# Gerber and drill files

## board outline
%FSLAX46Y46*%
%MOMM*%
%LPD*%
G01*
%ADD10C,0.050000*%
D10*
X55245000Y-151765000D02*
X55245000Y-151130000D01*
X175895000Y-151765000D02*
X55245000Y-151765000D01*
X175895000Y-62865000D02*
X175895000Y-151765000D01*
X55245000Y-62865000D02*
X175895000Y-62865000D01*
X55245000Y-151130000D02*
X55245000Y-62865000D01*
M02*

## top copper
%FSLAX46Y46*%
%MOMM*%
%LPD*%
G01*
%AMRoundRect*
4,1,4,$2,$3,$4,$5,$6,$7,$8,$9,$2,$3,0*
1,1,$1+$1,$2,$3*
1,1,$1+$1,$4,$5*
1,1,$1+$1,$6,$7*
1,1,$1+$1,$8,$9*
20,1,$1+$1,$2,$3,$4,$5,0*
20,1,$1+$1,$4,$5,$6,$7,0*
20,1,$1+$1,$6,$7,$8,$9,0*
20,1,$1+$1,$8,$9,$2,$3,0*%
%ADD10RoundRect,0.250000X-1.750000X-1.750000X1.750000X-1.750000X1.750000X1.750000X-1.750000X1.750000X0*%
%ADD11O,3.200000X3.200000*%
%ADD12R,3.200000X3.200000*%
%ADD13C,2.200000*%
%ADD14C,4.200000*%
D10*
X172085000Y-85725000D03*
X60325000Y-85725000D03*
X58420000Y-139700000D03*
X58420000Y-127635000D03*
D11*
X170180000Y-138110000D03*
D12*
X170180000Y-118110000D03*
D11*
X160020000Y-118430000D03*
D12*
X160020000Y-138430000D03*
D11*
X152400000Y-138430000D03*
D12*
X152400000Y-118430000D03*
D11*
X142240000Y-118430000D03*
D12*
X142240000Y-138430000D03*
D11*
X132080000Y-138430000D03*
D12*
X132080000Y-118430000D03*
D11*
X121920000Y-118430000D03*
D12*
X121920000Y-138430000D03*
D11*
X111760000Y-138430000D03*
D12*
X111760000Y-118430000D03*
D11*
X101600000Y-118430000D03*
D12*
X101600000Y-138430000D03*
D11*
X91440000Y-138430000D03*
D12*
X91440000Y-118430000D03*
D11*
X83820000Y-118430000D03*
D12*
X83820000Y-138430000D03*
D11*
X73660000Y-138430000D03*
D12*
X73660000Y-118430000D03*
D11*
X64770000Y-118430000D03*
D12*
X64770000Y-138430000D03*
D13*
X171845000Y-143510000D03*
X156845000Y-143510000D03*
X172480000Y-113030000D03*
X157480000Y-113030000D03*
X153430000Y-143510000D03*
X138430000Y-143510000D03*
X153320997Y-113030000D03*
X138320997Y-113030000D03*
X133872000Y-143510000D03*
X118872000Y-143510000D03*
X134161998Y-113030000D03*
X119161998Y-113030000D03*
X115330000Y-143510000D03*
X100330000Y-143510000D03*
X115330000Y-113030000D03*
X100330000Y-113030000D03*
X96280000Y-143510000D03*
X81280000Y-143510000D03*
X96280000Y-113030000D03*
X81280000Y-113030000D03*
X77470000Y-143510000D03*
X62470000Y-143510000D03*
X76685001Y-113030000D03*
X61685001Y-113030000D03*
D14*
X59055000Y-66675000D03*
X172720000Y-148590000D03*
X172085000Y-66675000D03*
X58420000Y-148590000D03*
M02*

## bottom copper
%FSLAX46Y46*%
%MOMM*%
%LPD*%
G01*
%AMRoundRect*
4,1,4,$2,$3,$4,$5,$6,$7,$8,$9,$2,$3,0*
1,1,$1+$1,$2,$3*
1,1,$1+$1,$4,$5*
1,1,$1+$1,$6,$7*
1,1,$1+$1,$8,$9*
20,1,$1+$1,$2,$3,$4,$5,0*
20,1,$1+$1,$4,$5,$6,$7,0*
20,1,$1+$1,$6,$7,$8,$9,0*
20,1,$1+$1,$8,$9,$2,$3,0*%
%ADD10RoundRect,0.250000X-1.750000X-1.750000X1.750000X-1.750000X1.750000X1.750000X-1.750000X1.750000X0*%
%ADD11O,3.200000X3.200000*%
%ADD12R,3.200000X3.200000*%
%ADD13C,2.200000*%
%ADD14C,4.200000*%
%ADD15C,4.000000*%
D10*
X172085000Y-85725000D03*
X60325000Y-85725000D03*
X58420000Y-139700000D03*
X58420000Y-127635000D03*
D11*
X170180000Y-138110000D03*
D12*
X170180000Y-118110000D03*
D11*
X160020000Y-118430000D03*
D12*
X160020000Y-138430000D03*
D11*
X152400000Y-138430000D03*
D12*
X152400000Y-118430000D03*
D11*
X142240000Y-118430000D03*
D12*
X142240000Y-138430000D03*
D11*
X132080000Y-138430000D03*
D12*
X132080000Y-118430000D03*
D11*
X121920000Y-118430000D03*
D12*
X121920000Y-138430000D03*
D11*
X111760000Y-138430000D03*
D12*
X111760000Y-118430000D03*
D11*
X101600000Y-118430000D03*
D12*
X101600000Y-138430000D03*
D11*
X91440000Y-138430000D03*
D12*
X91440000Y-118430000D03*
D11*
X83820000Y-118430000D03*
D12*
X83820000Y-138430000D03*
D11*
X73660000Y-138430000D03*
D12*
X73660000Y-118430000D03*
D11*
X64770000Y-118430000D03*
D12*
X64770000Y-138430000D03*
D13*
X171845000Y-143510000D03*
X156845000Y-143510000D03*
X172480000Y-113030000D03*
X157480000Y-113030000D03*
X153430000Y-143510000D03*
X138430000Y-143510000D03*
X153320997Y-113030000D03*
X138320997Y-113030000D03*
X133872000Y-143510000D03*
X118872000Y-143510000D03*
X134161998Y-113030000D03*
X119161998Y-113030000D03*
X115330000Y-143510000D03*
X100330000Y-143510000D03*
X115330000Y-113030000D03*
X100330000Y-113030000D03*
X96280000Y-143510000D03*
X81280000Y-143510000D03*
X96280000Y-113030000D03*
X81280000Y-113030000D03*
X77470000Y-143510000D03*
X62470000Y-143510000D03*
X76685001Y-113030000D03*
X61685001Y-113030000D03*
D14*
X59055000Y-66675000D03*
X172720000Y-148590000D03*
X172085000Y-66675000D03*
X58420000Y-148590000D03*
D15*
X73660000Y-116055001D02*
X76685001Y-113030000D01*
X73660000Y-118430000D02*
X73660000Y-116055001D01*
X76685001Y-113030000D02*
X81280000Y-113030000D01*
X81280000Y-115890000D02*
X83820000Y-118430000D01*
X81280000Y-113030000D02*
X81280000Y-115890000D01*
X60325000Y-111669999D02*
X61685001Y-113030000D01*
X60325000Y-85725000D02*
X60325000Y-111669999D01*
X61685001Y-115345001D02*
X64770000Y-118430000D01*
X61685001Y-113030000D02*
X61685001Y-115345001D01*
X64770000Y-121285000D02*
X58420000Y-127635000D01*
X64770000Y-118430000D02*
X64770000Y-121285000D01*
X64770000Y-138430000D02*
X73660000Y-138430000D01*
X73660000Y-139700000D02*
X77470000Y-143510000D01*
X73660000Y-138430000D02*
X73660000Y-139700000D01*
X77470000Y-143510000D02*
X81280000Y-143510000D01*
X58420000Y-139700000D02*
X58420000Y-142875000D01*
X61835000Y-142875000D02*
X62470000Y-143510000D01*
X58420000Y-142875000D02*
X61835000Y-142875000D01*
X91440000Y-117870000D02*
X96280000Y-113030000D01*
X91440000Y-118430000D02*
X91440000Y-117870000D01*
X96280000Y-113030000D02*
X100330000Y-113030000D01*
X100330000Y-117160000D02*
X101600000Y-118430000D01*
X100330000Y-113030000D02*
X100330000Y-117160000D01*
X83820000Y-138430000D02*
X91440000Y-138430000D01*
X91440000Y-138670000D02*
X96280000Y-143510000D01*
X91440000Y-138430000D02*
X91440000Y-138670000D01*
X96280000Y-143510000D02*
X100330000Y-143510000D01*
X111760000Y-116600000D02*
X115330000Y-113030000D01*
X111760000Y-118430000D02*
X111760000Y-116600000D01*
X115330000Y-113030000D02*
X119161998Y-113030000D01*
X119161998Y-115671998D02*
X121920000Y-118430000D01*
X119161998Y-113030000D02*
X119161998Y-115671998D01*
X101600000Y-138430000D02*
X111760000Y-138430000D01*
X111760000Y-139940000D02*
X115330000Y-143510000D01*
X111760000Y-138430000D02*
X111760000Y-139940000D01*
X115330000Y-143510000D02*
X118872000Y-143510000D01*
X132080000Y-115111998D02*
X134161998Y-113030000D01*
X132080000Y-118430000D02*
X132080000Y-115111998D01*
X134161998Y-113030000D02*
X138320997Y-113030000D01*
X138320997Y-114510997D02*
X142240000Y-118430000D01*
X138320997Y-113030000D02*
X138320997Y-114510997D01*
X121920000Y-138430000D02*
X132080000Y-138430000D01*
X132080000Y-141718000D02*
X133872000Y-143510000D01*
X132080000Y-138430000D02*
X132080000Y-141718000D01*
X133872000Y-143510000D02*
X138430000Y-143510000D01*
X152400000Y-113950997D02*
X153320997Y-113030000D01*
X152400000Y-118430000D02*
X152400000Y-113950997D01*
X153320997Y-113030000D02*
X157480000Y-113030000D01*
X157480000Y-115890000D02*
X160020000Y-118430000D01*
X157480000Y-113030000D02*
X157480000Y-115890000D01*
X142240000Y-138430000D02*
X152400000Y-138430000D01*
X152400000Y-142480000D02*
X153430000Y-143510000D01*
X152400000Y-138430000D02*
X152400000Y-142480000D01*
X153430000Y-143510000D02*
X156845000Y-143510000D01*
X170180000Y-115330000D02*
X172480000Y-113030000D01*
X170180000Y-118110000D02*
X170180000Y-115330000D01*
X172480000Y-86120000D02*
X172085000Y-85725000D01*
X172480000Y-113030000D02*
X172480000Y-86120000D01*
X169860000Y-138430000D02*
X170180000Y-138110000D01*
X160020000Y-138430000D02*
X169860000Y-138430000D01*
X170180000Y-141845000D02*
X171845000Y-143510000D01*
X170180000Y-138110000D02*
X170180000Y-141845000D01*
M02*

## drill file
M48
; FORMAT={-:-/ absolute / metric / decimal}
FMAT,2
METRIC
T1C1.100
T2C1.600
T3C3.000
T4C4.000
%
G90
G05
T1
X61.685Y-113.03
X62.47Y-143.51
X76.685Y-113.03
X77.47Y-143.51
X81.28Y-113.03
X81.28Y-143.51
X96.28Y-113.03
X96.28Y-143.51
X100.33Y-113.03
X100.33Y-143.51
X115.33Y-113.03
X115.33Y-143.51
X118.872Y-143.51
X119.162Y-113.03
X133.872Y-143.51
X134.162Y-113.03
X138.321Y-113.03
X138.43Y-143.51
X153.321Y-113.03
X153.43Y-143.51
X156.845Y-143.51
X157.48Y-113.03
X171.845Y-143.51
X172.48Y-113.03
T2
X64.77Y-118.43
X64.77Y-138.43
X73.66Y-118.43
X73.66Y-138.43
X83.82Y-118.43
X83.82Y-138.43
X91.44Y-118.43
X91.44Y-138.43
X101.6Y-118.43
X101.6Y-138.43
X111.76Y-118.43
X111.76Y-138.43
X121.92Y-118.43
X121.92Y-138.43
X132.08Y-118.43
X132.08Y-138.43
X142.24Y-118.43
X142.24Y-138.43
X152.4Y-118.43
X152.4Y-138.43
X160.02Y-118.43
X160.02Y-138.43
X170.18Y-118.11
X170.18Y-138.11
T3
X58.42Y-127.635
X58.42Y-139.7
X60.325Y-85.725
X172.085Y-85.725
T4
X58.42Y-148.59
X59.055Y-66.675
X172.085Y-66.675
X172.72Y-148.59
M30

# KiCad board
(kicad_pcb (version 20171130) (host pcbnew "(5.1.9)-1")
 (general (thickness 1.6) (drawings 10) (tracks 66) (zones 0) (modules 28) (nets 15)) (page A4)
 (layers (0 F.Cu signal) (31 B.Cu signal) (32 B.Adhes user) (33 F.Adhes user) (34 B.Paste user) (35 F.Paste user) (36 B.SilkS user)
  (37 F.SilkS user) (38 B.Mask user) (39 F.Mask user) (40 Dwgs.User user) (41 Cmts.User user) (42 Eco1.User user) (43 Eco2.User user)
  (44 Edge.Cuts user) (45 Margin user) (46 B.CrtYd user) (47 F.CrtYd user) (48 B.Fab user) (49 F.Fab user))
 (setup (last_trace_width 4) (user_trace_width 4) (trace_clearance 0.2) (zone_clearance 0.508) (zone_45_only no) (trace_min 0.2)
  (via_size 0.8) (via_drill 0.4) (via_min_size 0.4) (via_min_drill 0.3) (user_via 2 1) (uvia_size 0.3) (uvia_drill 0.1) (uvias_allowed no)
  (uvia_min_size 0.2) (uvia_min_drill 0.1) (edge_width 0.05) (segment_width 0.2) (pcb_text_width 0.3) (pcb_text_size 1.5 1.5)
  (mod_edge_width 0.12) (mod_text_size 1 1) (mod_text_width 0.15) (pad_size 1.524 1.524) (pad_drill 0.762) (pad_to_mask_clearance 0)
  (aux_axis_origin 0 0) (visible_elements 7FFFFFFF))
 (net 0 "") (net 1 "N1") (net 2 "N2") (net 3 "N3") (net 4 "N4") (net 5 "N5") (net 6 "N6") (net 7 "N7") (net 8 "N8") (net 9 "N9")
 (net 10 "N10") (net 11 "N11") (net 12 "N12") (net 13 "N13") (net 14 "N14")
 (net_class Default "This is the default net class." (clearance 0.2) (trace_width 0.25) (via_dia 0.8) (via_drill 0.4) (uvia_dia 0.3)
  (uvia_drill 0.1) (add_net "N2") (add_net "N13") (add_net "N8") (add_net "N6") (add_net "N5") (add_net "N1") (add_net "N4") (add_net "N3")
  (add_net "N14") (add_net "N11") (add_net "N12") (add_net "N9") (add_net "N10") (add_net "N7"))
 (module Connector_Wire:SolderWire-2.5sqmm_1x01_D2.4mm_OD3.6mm (layer F.Cu) (at 172.085 85.725)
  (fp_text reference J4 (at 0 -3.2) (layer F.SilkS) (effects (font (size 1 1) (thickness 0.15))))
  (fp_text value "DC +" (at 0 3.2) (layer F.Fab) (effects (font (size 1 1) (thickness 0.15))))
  (pad 1 thru_hole roundrect (at 0 0) (size 4 4) (drill 3) (layers *.Cu *.Mask) (roundrect_rratio 0.0625) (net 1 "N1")))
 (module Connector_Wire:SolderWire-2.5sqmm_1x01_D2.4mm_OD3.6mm (layer F.Cu) (at 60.325 85.725)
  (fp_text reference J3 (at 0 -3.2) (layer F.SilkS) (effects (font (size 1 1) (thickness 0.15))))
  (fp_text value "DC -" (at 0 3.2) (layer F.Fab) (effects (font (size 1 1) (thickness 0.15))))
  (pad 1 thru_hole roundrect (at 0 0) (size 4 4) (drill 3) (layers *.Cu *.Mask) (roundrect_rratio 0.0625) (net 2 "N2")))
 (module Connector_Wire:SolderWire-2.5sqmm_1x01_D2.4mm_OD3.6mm (layer F.Cu) (at 58.42 139.7)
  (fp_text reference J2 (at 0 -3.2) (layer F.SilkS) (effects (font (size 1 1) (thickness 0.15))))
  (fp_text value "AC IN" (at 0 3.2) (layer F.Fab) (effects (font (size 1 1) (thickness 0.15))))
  (pad 1 thru_hole roundrect (at 0 0) (size 4 4) (drill 3) (layers *.Cu *.Mask) (roundrect_rratio 0.0625) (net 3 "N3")))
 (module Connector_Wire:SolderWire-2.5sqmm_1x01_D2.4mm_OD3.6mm (layer F.Cu) (at 58.42 127.635)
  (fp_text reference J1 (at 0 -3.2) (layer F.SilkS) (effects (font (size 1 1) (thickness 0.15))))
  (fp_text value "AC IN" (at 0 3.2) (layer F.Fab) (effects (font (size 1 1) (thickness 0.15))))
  (pad 1 thru_hole roundrect (at 0 0) (size 4 4) (drill 3) (layers *.Cu *.Mask) (roundrect_rratio 0.0625) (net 2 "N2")))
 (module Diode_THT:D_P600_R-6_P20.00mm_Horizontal (layer F.Cu) (at 170.18 118.11 270)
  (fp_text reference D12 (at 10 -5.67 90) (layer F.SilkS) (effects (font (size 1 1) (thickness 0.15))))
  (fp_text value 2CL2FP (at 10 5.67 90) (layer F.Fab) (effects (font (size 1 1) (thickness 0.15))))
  (pad 2 thru_hole oval (at 20 0 270) (size 3.2 3.2) (drill 1.6) (layers *.Cu *.Mask) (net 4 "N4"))
  (pad 1 thru_hole rect (at 0 0 270) (size 3.2 3.2) (drill 1.6) (layers *.Cu *.Mask) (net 1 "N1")))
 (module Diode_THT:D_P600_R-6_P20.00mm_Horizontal (layer F.Cu) (at 160.02 138.43 90)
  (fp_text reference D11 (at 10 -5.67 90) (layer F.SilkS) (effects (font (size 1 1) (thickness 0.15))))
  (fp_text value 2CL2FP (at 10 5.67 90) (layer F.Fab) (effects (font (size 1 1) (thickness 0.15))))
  (pad 2 thru_hole oval (at 20 0 90) (size 3.2 3.2) (drill 1.6) (layers *.Cu *.Mask) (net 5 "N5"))
  (pad 1 thru_hole rect (at 0 0 90) (size 3.2 3.2) (drill 1.6) (layers *.Cu *.Mask) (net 4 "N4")))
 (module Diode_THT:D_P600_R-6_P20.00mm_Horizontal (layer F.Cu) (at 152.4 118.43 270)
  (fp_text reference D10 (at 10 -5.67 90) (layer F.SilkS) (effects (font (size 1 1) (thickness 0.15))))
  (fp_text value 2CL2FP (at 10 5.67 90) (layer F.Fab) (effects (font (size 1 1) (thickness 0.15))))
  (pad 2 thru_hole oval (at 20 0 270) (size 3.2 3.2) (drill 1.6) (layers *.Cu *.Mask) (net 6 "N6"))
  (pad 1 thru_hole rect (at 0 0 270) (size 3.2 3.2) (drill 1.6) (layers *.Cu *.Mask) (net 5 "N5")))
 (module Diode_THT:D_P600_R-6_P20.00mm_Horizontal (layer F.Cu) (at 142.24 138.43 90)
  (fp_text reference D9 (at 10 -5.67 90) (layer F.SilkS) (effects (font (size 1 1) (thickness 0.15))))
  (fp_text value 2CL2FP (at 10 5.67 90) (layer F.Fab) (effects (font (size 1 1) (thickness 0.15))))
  (pad 2 thru_hole oval (at 20 0 90) (size 3.2 3.2) (drill 1.6) (layers *.Cu *.Mask) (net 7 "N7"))
  (pad 1 thru_hole rect (at 0 0 90) (size 3.2 3.2) (drill 1.6) (layers *.Cu *.Mask) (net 6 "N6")))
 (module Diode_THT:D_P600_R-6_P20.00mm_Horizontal (layer F.Cu) (at 132.08 118.43 270)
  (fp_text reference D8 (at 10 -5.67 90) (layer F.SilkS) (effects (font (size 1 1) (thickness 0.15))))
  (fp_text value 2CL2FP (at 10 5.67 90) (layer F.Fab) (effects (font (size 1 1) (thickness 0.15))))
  (pad 2 thru_hole oval (at 20 0 270) (size 3.2 3.2) (drill 1.6) (layers *.Cu *.Mask) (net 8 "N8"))
  (pad 1 thru_hole rect (at 0 0 270) (size 3.2 3.2) (drill 1.6) (layers *.Cu *.Mask) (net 7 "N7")))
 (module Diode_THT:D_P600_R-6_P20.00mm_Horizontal (layer F.Cu) (at 121.92 138.43 90)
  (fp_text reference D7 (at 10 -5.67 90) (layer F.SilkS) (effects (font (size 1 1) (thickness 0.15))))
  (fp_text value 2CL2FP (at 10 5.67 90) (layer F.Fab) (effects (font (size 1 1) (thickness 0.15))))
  (pad 2 thru_hole oval (at 20 0 90) (size 3.2 3.2) (drill 1.6) (layers *.Cu *.Mask) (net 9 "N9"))
  (pad 1 thru_hole rect (at 0 0 90) (size 3.2 3.2) (drill 1.6) (layers *.Cu *.Mask) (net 8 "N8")))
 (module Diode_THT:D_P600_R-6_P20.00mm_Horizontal (layer F.Cu) (at 111.76 118.43 270)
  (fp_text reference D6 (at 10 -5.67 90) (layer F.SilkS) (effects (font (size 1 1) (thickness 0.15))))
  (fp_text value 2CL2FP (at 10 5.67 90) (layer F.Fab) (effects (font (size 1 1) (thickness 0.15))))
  (pad 2 thru_hole oval (at 20 0 270) (size 3.2 3.2) (drill 1.6) (layers *.Cu *.Mask) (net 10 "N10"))
  (pad 1 thru_hole rect (at 0 0 270) (size 3.2 3.2) (drill 1.6) (layers *.Cu *.Mask) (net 9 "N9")))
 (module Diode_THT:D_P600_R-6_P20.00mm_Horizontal (layer F.Cu) (at 101.6 138.43 90)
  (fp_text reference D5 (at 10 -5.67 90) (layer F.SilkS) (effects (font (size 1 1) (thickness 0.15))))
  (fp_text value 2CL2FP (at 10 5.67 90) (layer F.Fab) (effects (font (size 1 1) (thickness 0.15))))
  (pad 2 thru_hole oval (at 20 0 90) (size 3.2 3.2) (drill 1.6) (layers *.Cu *.Mask) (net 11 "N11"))
  (pad 1 thru_hole rect (at 0 0 90) (size 3.2 3.2) (drill 1.6) (layers *.Cu *.Mask) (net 10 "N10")))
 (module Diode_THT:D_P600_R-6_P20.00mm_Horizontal (layer F.Cu) (at 91.44 118.43 270)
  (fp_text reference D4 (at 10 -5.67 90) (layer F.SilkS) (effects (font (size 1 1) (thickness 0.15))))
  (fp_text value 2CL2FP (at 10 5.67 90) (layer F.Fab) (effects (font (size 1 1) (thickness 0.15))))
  (pad 2 thru_hole oval (at 20 0 270) (size 3.2 3.2) (drill 1.6) (layers *.Cu *.Mask) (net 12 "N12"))
  (pad 1 thru_hole rect (at 0 0 270) (size 3.2 3.2) (drill 1.6) (layers *.Cu *.Mask) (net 11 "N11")))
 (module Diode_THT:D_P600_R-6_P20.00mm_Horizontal (layer F.Cu) (at 83.82 138.43 90)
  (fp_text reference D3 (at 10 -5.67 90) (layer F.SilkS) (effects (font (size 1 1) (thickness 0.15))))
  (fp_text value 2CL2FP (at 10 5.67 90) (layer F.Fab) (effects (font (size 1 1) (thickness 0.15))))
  (pad 2 thru_hole oval (at 20 0 90) (size 3.2 3.2) (drill 1.6) (layers *.Cu *.Mask) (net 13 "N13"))
  (pad 1 thru_hole rect (at 0 0 90) (size 3.2 3.2) (drill 1.6) (layers *.Cu *.Mask) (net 12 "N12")))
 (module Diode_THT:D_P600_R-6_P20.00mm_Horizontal (layer F.Cu) (at 73.66 118.43 270)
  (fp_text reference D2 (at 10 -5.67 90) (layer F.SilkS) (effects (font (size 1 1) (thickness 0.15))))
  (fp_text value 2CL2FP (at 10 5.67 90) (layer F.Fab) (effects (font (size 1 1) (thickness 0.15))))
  (pad 2 thru_hole oval (at 20 0 270) (size 3.2 3.2) (drill 1.6) (layers *.Cu *.Mask) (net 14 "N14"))
  (pad 1 thru_hole rect (at 0 0 270) (size 3.2 3.2) (drill 1.6) (layers *.Cu *.Mask) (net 13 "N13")))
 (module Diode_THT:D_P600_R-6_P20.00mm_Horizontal (layer F.Cu) (at 64.77 138.43 90)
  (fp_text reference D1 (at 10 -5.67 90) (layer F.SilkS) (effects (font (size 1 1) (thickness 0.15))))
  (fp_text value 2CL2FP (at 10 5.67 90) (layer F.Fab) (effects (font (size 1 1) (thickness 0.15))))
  (pad 2 thru_hole oval (at 20 0 90) (size 3.2 3.2) (drill 1.6) (layers *.Cu *.Mask) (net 2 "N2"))
  (pad 1 thru_hole rect (at 0 0 90) (size 3.2 3.2) (drill 1.6) (layers *.Cu *.Mask) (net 14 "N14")))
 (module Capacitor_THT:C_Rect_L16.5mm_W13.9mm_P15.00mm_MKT (layer F.Cu) (at 156.845 143.51)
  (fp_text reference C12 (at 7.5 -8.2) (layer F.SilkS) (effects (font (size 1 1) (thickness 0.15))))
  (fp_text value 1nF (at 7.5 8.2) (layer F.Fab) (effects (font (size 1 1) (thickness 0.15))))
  (pad 2 thru_hole circle (at 15 0) (size 2.2 2.2) (drill 1.1) (layers *.Cu *.Mask) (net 4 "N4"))
  (pad 1 thru_hole circle (at 0 0) (size 2.2 2.2) (drill 1.1) (layers *.Cu *.Mask) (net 6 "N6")))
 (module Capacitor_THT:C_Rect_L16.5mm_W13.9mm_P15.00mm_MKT (layer F.Cu) (at 157.48 113.03)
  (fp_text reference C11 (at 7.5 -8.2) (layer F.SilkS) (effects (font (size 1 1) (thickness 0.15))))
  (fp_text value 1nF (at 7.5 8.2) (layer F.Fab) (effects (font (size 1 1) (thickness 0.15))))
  (pad 2 thru_hole circle (at 15 0) (size 2.2 2.2) (drill 1.1) (layers *.Cu *.Mask) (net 1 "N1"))
  (pad 1 thru_hole circle (at 0 0) (size 2.2 2.2) (drill 1.1) (layers *.Cu *.Mask) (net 5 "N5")))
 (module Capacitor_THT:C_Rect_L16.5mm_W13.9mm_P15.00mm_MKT (layer F.Cu) (at 138.43 143.51)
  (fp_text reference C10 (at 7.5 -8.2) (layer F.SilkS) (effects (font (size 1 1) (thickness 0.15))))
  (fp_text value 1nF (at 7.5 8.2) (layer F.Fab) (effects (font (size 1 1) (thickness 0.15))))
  (pad 2 thru_hole circle (at 15 0) (size 2.2 2.2) (drill 1.1) (layers *.Cu *.Mask) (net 6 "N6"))
  (pad 1 thru_hole circle (at 0 0) (size 2.2 2.2) (drill 1.1) (layers *.Cu *.Mask) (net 8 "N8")))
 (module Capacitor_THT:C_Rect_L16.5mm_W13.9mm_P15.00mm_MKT (layer F.Cu) (at 138.320997 113.03)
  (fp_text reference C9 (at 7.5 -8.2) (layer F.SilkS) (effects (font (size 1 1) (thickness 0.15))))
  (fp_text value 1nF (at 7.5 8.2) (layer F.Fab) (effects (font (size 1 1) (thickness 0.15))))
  (pad 2 thru_hole circle (at 15 0) (size 2.2 2.2) (drill 1.1) (layers *.Cu *.Mask) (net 5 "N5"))
  (pad 1 thru_hole circle (at 0 0) (size 2.2 2.2) (drill 1.1) (layers *.Cu *.Mask) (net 7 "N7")))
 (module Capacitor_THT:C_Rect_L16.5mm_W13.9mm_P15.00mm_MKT (layer F.Cu) (at 118.872 143.51)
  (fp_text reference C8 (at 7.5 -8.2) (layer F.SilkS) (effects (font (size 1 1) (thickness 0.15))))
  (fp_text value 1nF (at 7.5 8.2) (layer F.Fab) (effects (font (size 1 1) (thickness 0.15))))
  (pad 2 thru_hole circle (at 15 0) (size 2.2 2.2) (drill 1.1) (layers *.Cu *.Mask) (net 8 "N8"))
  (pad 1 thru_hole circle (at 0 0) (size 2.2 2.2) (drill 1.1) (layers *.Cu *.Mask) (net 10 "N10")))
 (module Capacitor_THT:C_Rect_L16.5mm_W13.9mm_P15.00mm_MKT (layer F.Cu) (at 119.161998 113.03)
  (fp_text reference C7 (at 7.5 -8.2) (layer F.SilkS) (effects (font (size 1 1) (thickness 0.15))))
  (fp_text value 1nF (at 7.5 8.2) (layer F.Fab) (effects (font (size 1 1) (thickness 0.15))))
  (pad 2 thru_hole circle (at 15 0) (size 2.2 2.2) (drill 1.1) (layers *.Cu *.Mask) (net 7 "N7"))
  (pad 1 thru_hole circle (at 0 0) (size 2.2 2.2) (drill 1.1) (layers *.Cu *.Mask) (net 9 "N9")))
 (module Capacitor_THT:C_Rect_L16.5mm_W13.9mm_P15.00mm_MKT (layer F.Cu) (at 100.33 143.51)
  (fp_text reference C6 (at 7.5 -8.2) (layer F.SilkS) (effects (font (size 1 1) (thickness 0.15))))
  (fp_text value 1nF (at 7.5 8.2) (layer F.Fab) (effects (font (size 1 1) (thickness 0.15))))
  (pad 2 thru_hole circle (at 15 0) (size 2.2 2.2) (drill 1.1) (layers *.Cu *.Mask) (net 10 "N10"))
  (pad 1 thru_hole circle (at 0 0) (size 2.2 2.2) (drill 1.1) (layers *.Cu *.Mask) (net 12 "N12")))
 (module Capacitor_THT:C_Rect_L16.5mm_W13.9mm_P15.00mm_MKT (layer F.Cu) (at 100.33 113.03)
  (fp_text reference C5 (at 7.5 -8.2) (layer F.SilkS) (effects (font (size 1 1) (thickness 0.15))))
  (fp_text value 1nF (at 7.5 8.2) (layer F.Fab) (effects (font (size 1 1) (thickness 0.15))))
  (pad 2 thru_hole circle (at 15 0) (size 2.2 2.2) (drill 1.1) (layers *.Cu *.Mask) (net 9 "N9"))
  (pad 1 thru_hole circle (at 0 0) (size 2.2 2.2) (drill 1.1) (layers *.Cu *.Mask) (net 11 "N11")))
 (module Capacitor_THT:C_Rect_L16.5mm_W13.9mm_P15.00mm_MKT (layer F.Cu) (at 81.28 143.51)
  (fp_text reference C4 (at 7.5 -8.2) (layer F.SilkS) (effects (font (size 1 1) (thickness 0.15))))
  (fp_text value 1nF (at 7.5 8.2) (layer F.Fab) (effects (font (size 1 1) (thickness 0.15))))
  (pad 2 thru_hole circle (at 15 0) (size 2.2 2.2) (drill 1.1) (layers *.Cu *.Mask) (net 12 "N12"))
  (pad 1 thru_hole circle (at 0 0) (size 2.2 2.2) (drill 1.1) (layers *.Cu *.Mask) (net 14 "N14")))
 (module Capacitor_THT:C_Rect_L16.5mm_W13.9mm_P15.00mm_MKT (layer F.Cu) (at 81.28 113.03)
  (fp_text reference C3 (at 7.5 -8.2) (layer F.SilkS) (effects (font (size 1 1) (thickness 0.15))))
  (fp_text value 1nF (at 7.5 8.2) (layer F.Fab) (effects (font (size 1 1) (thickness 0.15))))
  (pad 2 thru_hole circle (at 15 0) (size 2.2 2.2) (drill 1.1) (layers *.Cu *.Mask) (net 11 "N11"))
  (pad 1 thru_hole circle (at 0 0) (size 2.2 2.2) (drill 1.1) (layers *.Cu *.Mask) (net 13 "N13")))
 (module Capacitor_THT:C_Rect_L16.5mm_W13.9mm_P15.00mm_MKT (layer F.Cu) (at 62.47 143.51)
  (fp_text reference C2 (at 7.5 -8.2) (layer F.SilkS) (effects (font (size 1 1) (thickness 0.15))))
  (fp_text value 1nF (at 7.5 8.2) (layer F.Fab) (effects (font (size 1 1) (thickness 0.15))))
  (pad 2 thru_hole circle (at 15 0) (size 2.2 2.2) (drill 1.1) (layers *.Cu *.Mask) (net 14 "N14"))
  (pad 1 thru_hole circle (at 0 0) (size 2.2 2.2) (drill 1.1) (layers *.Cu *.Mask) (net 3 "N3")))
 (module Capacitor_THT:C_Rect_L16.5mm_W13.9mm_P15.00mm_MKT (layer F.Cu) (at 61.685001 113.03)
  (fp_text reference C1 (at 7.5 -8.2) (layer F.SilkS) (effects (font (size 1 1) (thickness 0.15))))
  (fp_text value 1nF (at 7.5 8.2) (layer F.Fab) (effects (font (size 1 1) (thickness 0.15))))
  (pad 2 thru_hole circle (at 15 0) (size 2.2 2.2) (drill 1.1) (layers *.Cu *.Mask) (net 13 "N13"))
  (pad 1 thru_hole circle (at 0 0) (size 2.2 2.2) (drill 1.1) (layers *.Cu *.Mask) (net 2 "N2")))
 (gr_line (start 55.245 151.765) (end 55.245 151.13) (layer Edge.Cuts) (width 0.05))
 (gr_line (start 175.895 151.765) (end 55.245 151.765) (layer Edge.Cuts) (width 0.05))
 (gr_line (start 175.895 62.865) (end 175.895 151.765) (layer Edge.Cuts) (width 0.05))
 (gr_line (start 55.245 62.865) (end 175.895 62.865) (layer Edge.Cuts) (width 0.05))
 (gr_line (start 55.245 151.13) (end 55.245 62.865) (layer Edge.Cuts) (width 0.05))
 (via (at 59.055 66.675) (size 4.2) (drill 4) (layers F.Cu B.Cu) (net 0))
 (via (at 172.72 148.59) (size 4.2) (drill 4) (layers F.Cu B.Cu) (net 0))
 (via (at 172.085 66.675) (size 4.2) (drill 4) (layers F.Cu B.Cu) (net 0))
 (via (at 58.42 148.59) (size 4.2) (drill 4) (layers F.Cu B.Cu) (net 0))
 (segment (start 73.66 116.055001) (end 76.685001 113.03) (width 4) (layer B.Cu) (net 13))
 (segment (start 73.66 118.43) (end 73.66 116.055001) (width 4) (layer B.Cu) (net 13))
 (segment (start 76.685001 113.03) (end 81.28 113.03) (width 4) (layer B.Cu) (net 13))
 (segment (start 81.28 115.89) (end 83.82 118.43) (width 4) (layer B.Cu) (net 13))
 (segment (start 81.28 113.03) (end 81.28 115.89) (width 4) (layer B.Cu) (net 13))
 (segment (start 60.325 111.669999) (end 61.685001 113.03) (width 4) (layer B.Cu) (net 2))
 (segment (start 60.325 85.725) (end 60.325 111.669999) (width 4) (layer B.Cu) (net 2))
 (segment (start 61.685001 115.345001) (end 64.77 118.43) (width 4) (layer B.Cu) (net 2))
 (segment (start 61.685001 113.03) (end 61.685001 115.345001) (width 4) (layer B.Cu) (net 2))
 (segment (start 64.77 121.285) (end 58.42 127.635) (width 4) (layer B.Cu) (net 2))
 (segment (start 64.77 118.43) (end 64.77 121.285) (width 4) (layer B.Cu) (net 2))
 (segment (start 64.77 138.43) (end 73.66 138.43) (width 4) (layer B.Cu) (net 14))
 (segment (start 73.66 139.7) (end 77.47 143.51) (width 4) (layer B.Cu) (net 14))
 (segment (start 73.66 138.43) (end 73.66 139.7) (width 4) (layer B.Cu) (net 14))
 (segment (start 77.47 143.51) (end 81.28 143.51) (width 4) (layer B.Cu) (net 14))
 (segment (start 58.42 139.7) (end 58.42 142.875) (width 4) (layer B.Cu) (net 3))
 (segment (start 61.835 142.875) (end 62.47 143.51) (width 4) (layer B.Cu) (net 3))
 (segment (start 58.42 142.875) (end 61.835 142.875) (width 4) (layer B.Cu) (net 3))
 (segment (start 91.44 117.87) (end 96.28 113.03) (width 4) (layer B.Cu) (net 11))
 (segment (start 91.44 118.43) (end 91.44 117.87) (width 4) (layer B.Cu) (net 11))
 (segment (start 96.28 113.03) (end 100.33 113.03) (width 4) (layer B.Cu) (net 11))
 (segment (start 100.33 117.16) (end 101.6 118.43) (width 4) (layer B.Cu) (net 11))
 (segment (start 100.33 113.03) (end 100.33 117.16) (width 4) (layer B.Cu) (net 11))
 (segment (start 83.82 138.43) (end 91.44 138.43) (width 4) (layer B.Cu) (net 12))
 (segment (start 91.44 138.67) (end 96.28 143.51) (width 4) (layer B.Cu) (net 12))
 (segment (start 91.44 138.43) (end 91.44 138.67) (width 4) (layer B.Cu) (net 12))
 (segment (start 96.28 143.51) (end 100.33 143.51) (width 4) (layer B.Cu) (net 12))
 (segment (start 111.76 116.6) (end 115.33 113.03) (width 4) (layer B.Cu) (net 9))
 (segment (start 111.76 118.43) (end 111.76 116.6) (width 4) (layer B.Cu) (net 9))
 (segment (start 115.33 113.03) (end 119.161998 113.03) (width 4) (layer B.Cu) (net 9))
 (segment (start 119.161998 115.671998) (end 121.92 118.43) (width 4) (layer B.Cu) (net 9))
 (segment (start 119.161998 113.03) (end 119.161998 115.671998) (width 4) (layer B.Cu) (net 9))
 (segment (start 101.6 138.43) (end 111.76 138.43) (width 4) (layer B.Cu) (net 10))
 (segment (start 111.76 139.94) (end 115.33 143.51) (width 4) (layer B.Cu) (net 10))
 (segment (start 111.76 138.43) (end 111.76 139.94) (width 4) (layer B.Cu) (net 10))
 (segment (start 115.33 143.51) (end 118.872 143.51) (width 4) (layer B.Cu) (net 10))
 (segment (start 132.08 115.111998) (end 134.161998 113.03) (width 4) (layer B.Cu) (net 7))
 (segment (start 132.08 118.43) (end 132.08 115.111998) (width 4) (layer B.Cu) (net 7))
 (segment (start 134.161998 113.03) (end 138.320997 113.03) (width 4) (layer B.Cu) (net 7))
 (segment (start 138.320997 114.510997) (end 142.24 118.43) (width 4) (layer B.Cu) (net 7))
 (segment (start 138.320997 113.03) (end 138.320997 114.510997) (width 4) (layer B.Cu) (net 7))
 (segment (start 121.92 138.43) (end 132.08 138.43) (width 4) (layer B.Cu) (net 8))
 (segment (start 132.08 141.718) (end 133.872 143.51) (width 4) (layer B.Cu) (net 8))
 (segment (start 132.08 138.43) (end 132.08 141.718) (width 4) (layer B.Cu) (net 8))
 (segment (start 133.872 143.51) (end 138.43 143.51) (width 4) (layer B.Cu) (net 8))
 (segment (start 152.4 113.950997) (end 153.320997 113.03) (width 4) (layer B.Cu) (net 5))
 (segment (start 152.4 118.43) (end 152.4 113.950997) (width 4) (layer B.Cu) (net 5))
 (segment (start 153.320997 113.03) (end 157.48 113.03) (width 4) (layer B.Cu) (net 5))
 (segment (start 157.48 115.89) (end 160.02 118.43) (width 4) (layer B.Cu) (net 5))
 (segment (start 157.48 113.03) (end 157.48 115.89) (width 4) (layer B.Cu) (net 5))
 (segment (start 142.24 138.43) (end 152.4 138.43) (width 4) (layer B.Cu) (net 6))
 (segment (start 152.4 142.48) (end 153.43 143.51) (width 4) (layer B.Cu) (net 6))
 (segment (start 152.4 138.43) (end 152.4 142.48) (width 4) (layer B.Cu) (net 6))
 (segment (start 153.43 143.51) (end 156.845 143.51) (width 4) (layer B.Cu) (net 6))
 (segment (start 170.18 115.33) (end 172.48 113.03) (width 4) (layer B.Cu) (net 1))
 (segment (start 170.18 118.11) (end 170.18 115.33) (width 4) (layer B.Cu) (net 1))
 (segment (start 172.48 86.12) (end 172.085 85.725) (width 4) (layer B.Cu) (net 1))
 (segment (start 172.48 113.03) (end 172.48 86.12) (width 4) (layer B.Cu) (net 1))
 (segment (start 169.86 138.43) (end 170.18 138.11) (width 4) (layer B.Cu) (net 4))
 (segment (start 160.02 138.43) (end 169.86 138.43) (width 4) (layer B.Cu) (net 4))
 (segment (start 170.18 141.845) (end 171.845 143.51) (width 4) (layer B.Cu) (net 4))
 (segment (start 170.18 138.11) (end 170.18 141.845) (width 4) (layer B.Cu) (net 4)))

